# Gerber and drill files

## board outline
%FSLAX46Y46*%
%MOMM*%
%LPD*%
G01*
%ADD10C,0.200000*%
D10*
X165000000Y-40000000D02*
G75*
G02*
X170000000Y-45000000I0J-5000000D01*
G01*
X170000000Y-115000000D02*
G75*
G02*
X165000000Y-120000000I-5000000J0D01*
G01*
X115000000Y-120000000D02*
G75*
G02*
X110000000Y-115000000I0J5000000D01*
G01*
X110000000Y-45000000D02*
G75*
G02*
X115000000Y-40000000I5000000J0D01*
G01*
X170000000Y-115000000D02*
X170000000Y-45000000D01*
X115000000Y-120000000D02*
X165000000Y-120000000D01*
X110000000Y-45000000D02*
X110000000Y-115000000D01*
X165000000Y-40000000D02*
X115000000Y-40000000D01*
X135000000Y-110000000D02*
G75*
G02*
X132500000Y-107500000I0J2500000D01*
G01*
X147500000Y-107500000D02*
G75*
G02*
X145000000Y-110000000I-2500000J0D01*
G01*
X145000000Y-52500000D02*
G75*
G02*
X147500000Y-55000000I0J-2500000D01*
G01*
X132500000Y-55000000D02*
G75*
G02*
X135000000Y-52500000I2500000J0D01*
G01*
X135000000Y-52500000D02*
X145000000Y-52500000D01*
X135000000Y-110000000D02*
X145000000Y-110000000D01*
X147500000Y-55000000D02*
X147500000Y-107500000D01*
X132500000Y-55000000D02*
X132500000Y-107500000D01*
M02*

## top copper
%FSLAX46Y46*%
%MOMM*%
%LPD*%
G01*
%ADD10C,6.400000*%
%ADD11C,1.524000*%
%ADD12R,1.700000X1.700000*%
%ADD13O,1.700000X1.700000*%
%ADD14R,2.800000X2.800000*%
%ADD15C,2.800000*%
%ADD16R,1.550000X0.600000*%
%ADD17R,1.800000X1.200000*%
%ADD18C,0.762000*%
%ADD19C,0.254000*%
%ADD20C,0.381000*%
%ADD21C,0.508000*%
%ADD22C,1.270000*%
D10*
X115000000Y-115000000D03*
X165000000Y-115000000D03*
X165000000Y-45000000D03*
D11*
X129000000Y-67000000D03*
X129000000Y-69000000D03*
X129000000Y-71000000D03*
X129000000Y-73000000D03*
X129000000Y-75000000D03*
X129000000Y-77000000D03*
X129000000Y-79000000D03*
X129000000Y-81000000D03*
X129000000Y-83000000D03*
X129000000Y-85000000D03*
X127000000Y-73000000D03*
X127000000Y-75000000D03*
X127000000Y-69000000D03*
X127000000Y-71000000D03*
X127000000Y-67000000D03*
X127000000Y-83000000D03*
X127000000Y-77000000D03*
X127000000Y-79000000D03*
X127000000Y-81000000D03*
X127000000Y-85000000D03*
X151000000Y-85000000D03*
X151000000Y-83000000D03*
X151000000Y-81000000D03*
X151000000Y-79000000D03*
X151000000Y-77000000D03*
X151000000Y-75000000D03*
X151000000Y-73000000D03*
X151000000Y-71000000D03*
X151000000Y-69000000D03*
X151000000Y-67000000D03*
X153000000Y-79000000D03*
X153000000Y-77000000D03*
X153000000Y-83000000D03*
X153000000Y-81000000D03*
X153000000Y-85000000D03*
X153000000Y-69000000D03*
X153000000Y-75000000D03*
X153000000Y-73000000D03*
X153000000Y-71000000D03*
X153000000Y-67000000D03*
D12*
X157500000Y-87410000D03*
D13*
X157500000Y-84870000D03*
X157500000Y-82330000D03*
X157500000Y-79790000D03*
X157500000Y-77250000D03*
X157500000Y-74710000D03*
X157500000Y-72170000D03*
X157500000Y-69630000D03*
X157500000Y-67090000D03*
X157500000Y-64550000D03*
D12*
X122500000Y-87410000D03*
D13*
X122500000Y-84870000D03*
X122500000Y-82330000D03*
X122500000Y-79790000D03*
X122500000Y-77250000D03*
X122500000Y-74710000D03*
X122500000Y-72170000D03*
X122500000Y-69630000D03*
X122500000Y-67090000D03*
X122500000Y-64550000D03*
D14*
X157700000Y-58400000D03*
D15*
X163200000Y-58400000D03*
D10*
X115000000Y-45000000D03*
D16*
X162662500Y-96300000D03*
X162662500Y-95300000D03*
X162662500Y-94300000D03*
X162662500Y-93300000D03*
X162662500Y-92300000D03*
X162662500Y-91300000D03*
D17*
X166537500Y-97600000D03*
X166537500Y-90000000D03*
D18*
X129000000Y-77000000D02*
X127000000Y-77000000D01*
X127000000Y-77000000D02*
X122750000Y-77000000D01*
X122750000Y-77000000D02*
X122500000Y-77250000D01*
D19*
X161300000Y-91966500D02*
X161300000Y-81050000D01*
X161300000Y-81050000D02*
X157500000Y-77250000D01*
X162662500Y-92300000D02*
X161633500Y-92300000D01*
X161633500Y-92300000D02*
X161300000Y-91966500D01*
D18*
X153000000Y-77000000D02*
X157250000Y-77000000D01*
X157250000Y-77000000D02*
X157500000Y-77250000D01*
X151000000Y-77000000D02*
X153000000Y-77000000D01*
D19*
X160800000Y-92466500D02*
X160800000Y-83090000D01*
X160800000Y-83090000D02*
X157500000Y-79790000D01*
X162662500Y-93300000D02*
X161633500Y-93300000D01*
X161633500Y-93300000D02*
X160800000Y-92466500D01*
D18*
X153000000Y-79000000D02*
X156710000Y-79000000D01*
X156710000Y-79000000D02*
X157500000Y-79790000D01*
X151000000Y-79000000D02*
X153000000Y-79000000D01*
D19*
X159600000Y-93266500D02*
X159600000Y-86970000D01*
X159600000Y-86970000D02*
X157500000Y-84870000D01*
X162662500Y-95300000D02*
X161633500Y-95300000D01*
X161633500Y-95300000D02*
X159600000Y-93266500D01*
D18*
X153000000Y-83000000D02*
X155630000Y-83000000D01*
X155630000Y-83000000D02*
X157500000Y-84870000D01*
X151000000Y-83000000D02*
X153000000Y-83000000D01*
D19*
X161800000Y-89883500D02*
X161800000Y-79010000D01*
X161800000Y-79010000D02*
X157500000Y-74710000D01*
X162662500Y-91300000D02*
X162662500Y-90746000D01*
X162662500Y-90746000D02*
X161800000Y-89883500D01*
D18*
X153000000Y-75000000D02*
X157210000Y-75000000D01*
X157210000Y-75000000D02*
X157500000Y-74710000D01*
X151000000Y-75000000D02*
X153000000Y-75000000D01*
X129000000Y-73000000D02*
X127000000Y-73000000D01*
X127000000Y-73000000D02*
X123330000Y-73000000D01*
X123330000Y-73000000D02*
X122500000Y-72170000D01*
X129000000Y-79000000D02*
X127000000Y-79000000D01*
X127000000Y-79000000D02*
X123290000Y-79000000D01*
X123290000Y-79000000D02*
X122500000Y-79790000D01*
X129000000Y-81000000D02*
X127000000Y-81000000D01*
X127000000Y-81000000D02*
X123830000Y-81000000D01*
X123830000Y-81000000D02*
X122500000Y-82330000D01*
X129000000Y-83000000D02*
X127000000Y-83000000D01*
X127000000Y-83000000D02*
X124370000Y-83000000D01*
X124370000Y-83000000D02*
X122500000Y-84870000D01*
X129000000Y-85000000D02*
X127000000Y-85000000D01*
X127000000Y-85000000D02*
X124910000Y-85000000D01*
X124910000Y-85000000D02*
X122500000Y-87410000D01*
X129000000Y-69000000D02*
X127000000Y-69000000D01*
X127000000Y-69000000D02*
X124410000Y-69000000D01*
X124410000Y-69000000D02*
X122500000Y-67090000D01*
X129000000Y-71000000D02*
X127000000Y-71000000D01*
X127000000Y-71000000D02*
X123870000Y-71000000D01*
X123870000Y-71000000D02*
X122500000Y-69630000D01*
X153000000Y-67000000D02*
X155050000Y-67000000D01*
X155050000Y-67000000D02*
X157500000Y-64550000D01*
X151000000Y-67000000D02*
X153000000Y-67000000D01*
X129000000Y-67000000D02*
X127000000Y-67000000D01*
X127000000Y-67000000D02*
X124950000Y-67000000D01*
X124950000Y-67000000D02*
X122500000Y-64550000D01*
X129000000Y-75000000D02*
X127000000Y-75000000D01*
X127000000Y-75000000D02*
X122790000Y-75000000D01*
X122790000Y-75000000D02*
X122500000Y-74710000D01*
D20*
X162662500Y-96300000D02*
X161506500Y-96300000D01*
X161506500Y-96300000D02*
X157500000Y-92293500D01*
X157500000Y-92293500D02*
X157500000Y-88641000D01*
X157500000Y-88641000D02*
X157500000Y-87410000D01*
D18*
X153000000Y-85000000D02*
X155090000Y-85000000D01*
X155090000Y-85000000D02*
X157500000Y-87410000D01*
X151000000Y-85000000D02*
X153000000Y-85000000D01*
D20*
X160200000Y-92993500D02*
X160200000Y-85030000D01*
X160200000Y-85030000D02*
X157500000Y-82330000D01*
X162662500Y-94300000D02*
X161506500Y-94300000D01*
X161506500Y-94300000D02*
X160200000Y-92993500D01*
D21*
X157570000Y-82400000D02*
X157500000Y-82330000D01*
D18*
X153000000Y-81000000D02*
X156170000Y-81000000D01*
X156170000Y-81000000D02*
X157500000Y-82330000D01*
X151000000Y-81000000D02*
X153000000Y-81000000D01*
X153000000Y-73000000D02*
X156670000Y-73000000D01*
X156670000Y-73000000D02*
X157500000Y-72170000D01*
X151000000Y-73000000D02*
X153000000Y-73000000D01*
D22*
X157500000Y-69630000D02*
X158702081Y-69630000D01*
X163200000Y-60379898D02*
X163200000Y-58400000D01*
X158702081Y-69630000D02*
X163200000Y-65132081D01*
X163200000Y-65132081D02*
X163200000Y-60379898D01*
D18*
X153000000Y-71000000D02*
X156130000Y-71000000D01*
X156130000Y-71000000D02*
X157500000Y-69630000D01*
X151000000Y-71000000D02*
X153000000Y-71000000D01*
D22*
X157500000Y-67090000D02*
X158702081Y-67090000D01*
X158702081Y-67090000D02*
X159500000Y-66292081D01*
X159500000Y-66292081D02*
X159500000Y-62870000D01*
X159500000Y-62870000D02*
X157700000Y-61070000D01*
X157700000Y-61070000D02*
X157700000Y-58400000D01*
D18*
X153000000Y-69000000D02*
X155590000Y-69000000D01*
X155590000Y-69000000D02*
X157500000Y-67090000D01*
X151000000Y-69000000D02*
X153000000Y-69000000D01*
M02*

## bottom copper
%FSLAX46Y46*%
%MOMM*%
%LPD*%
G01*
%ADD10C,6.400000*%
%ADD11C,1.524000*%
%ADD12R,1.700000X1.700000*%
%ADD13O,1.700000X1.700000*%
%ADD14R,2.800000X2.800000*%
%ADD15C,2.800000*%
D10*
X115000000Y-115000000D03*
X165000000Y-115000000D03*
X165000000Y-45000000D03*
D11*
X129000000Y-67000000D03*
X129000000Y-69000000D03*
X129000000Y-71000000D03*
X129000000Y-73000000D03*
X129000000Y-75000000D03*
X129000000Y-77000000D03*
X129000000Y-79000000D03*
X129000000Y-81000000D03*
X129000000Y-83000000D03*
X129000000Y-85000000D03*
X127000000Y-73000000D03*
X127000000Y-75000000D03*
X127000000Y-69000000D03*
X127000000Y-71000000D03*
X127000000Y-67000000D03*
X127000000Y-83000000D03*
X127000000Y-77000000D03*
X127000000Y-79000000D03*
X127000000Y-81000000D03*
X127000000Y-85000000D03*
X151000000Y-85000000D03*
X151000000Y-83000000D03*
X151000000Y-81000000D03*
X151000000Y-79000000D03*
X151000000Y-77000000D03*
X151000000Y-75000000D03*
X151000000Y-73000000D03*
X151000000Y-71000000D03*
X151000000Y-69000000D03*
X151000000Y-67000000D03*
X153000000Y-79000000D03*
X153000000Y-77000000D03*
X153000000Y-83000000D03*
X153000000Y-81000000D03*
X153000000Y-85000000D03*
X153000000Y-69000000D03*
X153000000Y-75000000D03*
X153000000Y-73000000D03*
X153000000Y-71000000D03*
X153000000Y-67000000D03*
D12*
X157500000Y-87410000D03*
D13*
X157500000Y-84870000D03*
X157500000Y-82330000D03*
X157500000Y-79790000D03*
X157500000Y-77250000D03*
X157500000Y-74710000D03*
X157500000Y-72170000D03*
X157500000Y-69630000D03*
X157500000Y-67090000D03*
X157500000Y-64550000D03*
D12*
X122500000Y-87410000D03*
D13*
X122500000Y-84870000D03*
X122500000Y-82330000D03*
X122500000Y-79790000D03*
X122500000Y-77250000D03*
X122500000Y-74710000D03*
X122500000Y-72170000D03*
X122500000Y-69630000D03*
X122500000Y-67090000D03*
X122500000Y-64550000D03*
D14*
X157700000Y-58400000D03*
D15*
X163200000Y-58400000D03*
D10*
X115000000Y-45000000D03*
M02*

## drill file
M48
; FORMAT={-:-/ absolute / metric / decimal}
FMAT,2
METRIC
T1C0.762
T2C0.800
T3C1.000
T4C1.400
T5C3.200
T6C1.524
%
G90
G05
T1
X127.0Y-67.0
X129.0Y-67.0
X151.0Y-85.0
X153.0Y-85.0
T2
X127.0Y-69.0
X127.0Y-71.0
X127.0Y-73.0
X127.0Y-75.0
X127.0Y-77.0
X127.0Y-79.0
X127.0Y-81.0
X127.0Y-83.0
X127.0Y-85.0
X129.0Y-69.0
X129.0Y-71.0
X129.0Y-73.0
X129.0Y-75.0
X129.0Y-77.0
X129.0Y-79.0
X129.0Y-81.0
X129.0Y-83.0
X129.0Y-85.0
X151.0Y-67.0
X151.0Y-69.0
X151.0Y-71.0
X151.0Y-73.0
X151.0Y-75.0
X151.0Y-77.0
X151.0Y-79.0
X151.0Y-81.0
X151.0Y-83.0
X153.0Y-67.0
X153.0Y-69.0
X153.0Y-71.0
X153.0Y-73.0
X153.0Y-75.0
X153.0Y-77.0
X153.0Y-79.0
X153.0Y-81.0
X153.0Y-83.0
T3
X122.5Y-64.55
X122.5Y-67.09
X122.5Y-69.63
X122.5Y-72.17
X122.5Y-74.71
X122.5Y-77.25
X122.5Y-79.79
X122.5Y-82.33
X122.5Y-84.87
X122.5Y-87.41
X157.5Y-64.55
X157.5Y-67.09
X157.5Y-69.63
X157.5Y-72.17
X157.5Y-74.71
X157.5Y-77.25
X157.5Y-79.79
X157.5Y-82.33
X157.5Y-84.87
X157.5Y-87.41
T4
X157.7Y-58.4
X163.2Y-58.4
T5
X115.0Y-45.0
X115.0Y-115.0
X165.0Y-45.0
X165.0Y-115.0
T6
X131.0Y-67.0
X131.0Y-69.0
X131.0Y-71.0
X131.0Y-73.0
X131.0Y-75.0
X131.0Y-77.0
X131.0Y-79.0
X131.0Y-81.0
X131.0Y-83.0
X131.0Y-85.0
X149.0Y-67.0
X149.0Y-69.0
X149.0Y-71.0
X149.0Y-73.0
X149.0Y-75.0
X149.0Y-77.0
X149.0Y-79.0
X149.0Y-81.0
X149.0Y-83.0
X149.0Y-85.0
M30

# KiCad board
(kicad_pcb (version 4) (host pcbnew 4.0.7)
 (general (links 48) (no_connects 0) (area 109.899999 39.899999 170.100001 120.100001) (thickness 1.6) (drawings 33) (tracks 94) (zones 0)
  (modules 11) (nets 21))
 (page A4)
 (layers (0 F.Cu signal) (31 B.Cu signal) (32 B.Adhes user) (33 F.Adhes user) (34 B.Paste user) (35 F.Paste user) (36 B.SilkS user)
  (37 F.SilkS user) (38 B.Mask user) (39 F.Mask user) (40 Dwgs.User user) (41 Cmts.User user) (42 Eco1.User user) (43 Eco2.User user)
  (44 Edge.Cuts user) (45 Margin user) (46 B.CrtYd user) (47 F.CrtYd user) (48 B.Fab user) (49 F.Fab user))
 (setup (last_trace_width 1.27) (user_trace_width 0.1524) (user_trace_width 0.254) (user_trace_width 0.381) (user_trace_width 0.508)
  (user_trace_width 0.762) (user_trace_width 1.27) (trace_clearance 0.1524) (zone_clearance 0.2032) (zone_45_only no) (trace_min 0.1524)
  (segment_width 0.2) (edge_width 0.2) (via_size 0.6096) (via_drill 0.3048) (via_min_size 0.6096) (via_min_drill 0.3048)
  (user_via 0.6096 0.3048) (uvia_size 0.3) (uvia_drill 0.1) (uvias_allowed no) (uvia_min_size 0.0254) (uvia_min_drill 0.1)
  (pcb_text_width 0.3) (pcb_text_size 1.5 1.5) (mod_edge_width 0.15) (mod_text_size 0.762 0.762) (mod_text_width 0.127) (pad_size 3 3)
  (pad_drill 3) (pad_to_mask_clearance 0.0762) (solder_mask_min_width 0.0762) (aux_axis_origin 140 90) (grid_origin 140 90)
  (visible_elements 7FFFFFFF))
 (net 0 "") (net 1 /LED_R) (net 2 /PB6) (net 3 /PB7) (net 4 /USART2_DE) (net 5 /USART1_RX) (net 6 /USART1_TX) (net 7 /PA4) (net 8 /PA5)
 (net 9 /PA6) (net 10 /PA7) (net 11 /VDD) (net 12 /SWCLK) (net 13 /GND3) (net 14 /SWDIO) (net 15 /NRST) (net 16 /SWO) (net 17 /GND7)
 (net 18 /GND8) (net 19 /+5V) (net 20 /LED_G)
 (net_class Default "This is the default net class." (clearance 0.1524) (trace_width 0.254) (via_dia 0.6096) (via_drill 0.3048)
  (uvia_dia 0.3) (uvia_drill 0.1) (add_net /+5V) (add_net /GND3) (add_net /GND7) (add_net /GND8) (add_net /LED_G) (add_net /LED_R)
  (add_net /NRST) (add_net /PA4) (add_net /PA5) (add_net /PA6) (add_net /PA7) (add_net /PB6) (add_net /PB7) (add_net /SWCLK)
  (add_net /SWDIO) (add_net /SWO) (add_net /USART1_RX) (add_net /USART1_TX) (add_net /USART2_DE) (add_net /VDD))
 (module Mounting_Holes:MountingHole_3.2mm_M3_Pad (layer F.Cu) (at 115 115)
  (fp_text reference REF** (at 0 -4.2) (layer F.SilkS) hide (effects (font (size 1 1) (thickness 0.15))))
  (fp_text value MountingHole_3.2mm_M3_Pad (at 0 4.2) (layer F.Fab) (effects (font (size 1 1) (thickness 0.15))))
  (pad 1 thru_hole circle (at 0 0) (size 6.4 6.4) (drill 3.2) (layers *.Cu *.Mask)))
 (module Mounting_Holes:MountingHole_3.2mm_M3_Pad (layer F.Cu) (at 165 115)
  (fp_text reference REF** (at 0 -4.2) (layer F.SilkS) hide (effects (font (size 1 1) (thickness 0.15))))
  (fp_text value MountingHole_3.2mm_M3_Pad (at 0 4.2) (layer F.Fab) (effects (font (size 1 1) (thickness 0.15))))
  (pad 1 thru_hole circle (at 0 0) (size 6.4 6.4) (drill 3.2) (layers *.Cu *.Mask)))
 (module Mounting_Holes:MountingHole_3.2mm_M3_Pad (layer F.Cu) (at 165 45)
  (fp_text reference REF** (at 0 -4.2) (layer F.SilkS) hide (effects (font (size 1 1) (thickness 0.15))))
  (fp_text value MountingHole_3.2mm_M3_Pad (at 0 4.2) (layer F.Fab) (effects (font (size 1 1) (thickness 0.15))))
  (pad 1 thru_hole circle (at 0 0) (size 6.4 6.4) (drill 3.2) (layers *.Cu *.Mask)))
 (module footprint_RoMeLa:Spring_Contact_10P (layer F.Cu) (at 129 67 180)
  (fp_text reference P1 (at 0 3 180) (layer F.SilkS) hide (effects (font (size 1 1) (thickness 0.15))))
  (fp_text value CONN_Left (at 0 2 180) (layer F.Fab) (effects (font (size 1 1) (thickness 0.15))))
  (pad 1 thru_hole circle (at 0 0 180) (size 1.524 1.524) (drill 0.762) (layers *.Cu *.Mask) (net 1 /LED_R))
  (pad 2 thru_hole circle (at 0 -2 180) (size 1.524 1.524) (drill 0.8) (layers *.Cu *.Mask) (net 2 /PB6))
  (pad 3 thru_hole circle (at 0 -4 180) (size 1.524 1.524) (drill 0.8) (layers *.Cu *.Mask) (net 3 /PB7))
  (pad 4 thru_hole circle (at 0 -6 180) (size 1.524 1.524) (drill 0.8) (layers *.Cu *.Mask) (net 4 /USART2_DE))
  (pad 5 thru_hole circle (at 0 -8 180) (size 1.524 1.524) (drill 0.8) (layers *.Cu *.Mask) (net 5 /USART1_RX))
  (pad 6 thru_hole circle (at 0 -10 180) (size 1.524 1.524) (drill 0.8) (layers *.Cu *.Mask) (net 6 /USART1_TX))
  (pad 7 thru_hole circle (at 0 -12 180) (size 1.524 1.524) (drill 0.8) (layers *.Cu *.Mask) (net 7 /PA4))
  (pad 8 thru_hole circle (at 0 -14 180) (size 1.524 1.524) (drill 0.8) (layers *.Cu *.Mask) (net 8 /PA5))
  (pad 9 thru_hole circle (at 0 -16 180) (size 1.524 1.524) (drill 0.8) (layers *.Cu *.Mask) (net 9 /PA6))
  (pad 10 thru_hole circle (at 0 -18 180) (size 1.524 1.524) (drill 0.8) (layers *.Cu *.Mask) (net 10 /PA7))
  (pad 4 thru_hole circle (at 2 -6 180) (size 1.524 1.524) (drill 0.8) (layers *.Cu *.Mask) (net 4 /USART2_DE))
  (pad 5 thru_hole circle (at 2 -8 180) (size 1.524 1.524) (drill 0.8) (layers *.Cu *.Mask) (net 5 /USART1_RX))
  (pad 2 thru_hole circle (at 2 -2 180) (size 1.524 1.524) (drill 0.8) (layers *.Cu *.Mask) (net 2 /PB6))
  (pad 3 thru_hole circle (at 2 -4 180) (size 1.524 1.524) (drill 0.8) (layers *.Cu *.Mask) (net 3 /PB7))
  (pad 1 thru_hole circle (at 2 0 180) (size 1.524 1.524) (drill 0.762) (layers *.Cu *.Mask) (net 1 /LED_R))
  (pad 9 thru_hole circle (at 2 -16 180) (size 1.524 1.524) (drill 0.8) (layers *.Cu *.Mask) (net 9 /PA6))
  (pad 6 thru_hole circle (at 2 -10 180) (size 1.524 1.524) (drill 0.8) (layers *.Cu *.Mask) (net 6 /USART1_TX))
  (pad 7 thru_hole circle (at 2 -12 180) (size 1.524 1.524) (drill 0.8) (layers *.Cu *.Mask) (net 7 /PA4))
  (pad 8 thru_hole circle (at 2 -14 180) (size 1.524 1.524) (drill 0.8) (layers *.Cu *.Mask) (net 8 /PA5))
  (pad 10 thru_hole circle (at 2 -18 180) (size 1.524 1.524) (drill 0.8) (layers *.Cu *.Mask) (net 10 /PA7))
  (pad "" np_thru_hole circle (at -2 0 180) (size 1.524 1.524) (drill 1.524) (layers *.Cu *.Mask))
  (pad "" np_thru_hole circle (at -2 -2 180) (size 1.524 1.524) (drill 1.524) (layers *.Cu *.Mask))
  (pad "" np_thru_hole circle (at -2 -4 180) (size 1.524 1.524) (drill 1.524) (layers *.Cu *.Mask))
  (pad "" np_thru_hole circle (at -2 -6 180) (size 1.524 1.524) (drill 1.524) (layers *.Cu *.Mask))
  (pad "" np_thru_hole circle (at -2 -8 180) (size 1.524 1.524) (drill 1.524) (layers *.Cu *.Mask))
  (pad "" np_thru_hole circle (at -2 -10 180) (size 1.524 1.524) (drill 1.524) (layers *.Cu *.Mask))
  (pad "" np_thru_hole circle (at -2 -12 180) (size 1.524 1.524) (drill 1.524) (layers *.Cu *.Mask))
  (pad "" np_thru_hole circle (at -2 -14 180) (size 1.524 1.524) (drill 1.524) (layers *.Cu *.Mask))
  (pad "" np_thru_hole circle (at -2 -16 180) (size 1.524 1.524) (drill 1.524) (layers *.Cu *.Mask))
  (pad "" np_thru_hole circle (at -2 -18 180) (size 1.524 1.524) (drill 1.524) (layers *.Cu *.Mask)))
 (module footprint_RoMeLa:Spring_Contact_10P (layer F.Cu) (at 151 85)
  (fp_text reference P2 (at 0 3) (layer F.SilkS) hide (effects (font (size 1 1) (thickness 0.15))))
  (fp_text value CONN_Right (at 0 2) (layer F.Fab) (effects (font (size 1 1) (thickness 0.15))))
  (pad 1 thru_hole circle (at 0 0) (size 1.524 1.524) (drill 0.762) (layers *.Cu *.Mask) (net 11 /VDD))
  (pad 2 thru_hole circle (at 0 -2) (size 1.524 1.524) (drill 0.8) (layers *.Cu *.Mask) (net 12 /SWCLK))
  (pad 3 thru_hole circle (at 0 -4) (size 1.524 1.524) (drill 0.8) (layers *.Cu *.Mask) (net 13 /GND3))
  (pad 4 thru_hole circle (at 0 -6) (size 1.524 1.524) (drill 0.8) (layers *.Cu *.Mask) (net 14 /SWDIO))
  (pad 5 thru_hole circle (at 0 -8) (size 1.524 1.524) (drill 0.8) (layers *.Cu *.Mask) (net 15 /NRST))
  (pad 6 thru_hole circle (at 0 -10) (size 1.524 1.524) (drill 0.8) (layers *.Cu *.Mask) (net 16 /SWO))
  (pad 7 thru_hole circle (at 0 -12) (size 1.524 1.524) (drill 0.8) (layers *.Cu *.Mask) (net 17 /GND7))
  (pad 8 thru_hole circle (at 0 -14) (size 1.524 1.524) (drill 0.8) (layers *.Cu *.Mask) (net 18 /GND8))
  (pad 9 thru_hole circle (at 0 -16) (size 1.524 1.524) (drill 0.8) (layers *.Cu *.Mask) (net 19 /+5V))
  (pad 10 thru_hole circle (at 0 -18) (size 1.524 1.524) (drill 0.8) (layers *.Cu *.Mask) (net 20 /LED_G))
  (pad 4 thru_hole circle (at 2 -6) (size 1.524 1.524) (drill 0.8) (layers *.Cu *.Mask) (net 14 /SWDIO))
  (pad 5 thru_hole circle (at 2 -8) (size 1.524 1.524) (drill 0.8) (layers *.Cu *.Mask) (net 15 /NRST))
  (pad 2 thru_hole circle (at 2 -2) (size 1.524 1.524) (drill 0.8) (layers *.Cu *.Mask) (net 12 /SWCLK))
  (pad 3 thru_hole circle (at 2 -4) (size 1.524 1.524) (drill 0.8) (layers *.Cu *.Mask) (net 13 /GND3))
  (pad 1 thru_hole circle (at 2 0) (size 1.524 1.524) (drill 0.762) (layers *.Cu *.Mask) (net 11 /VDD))
  (pad 9 thru_hole circle (at 2 -16) (size 1.524 1.524) (drill 0.8) (layers *.Cu *.Mask) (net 19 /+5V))
  (pad 6 thru_hole circle (at 2 -10) (size 1.524 1.524) (drill 0.8) (layers *.Cu *.Mask) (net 16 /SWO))
  (pad 7 thru_hole circle (at 2 -12) (size 1.524 1.524) (drill 0.8) (layers *.Cu *.Mask) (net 17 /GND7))
  (pad 8 thru_hole circle (at 2 -14) (size 1.524 1.524) (drill 0.8) (layers *.Cu *.Mask) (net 18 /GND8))
  (pad 10 thru_hole circle (at 2 -18) (size 1.524 1.524) (drill 0.8) (layers *.Cu *.Mask) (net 20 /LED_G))
  (pad "" np_thru_hole circle (at -2 0) (size 1.524 1.524) (drill 1.524) (layers *.Cu *.Mask))
  (pad "" np_thru_hole circle (at -2 -2) (size 1.524 1.524) (drill 1.524) (layers *.Cu *.Mask))
  (pad "" np_thru_hole circle (at -2 -4) (size 1.524 1.524) (drill 1.524) (layers *.Cu *.Mask))
  (pad "" np_thru_hole circle (at -2 -6) (size 1.524 1.524) (drill 1.524) (layers *.Cu *.Mask))
  (pad "" np_thru_hole circle (at -2 -8) (size 1.524 1.524) (drill 1.524) (layers *.Cu *.Mask))
  (pad "" np_thru_hole circle (at -2 -10) (size 1.524 1.524) (drill 1.524) (layers *.Cu *.Mask))
  (pad "" np_thru_hole circle (at -2 -12) (size 1.524 1.524) (drill 1.524) (layers *.Cu *.Mask))
  (pad "" np_thru_hole circle (at -2 -14) (size 1.524 1.524) (drill 1.524) (layers *.Cu *.Mask))
  (pad "" np_thru_hole circle (at -2 -16) (size 1.524 1.524) (drill 1.524) (layers *.Cu *.Mask))
  (pad "" np_thru_hole circle (at -2 -18) (size 1.524 1.524) (drill 1.524) (layers *.Cu *.Mask)))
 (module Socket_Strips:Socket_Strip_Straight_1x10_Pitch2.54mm (layer F.Cu) (at 157.5 87.41 180)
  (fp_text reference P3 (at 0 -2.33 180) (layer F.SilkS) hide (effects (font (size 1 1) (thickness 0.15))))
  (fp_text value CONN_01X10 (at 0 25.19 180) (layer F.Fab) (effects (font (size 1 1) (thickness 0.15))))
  (pad 1 thru_hole rect (at 0 0 180) (size 1.7 1.7) (drill 1) (layers *.Cu *.Mask) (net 11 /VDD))
  (pad 2 thru_hole oval (at 0 2.54 180) (size 1.7 1.7) (drill 1) (layers *.Cu *.Mask) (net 12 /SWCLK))
  (pad 3 thru_hole oval (at 0 5.08 180) (size 1.7 1.7) (drill 1) (layers *.Cu *.Mask) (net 13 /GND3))
  (pad 4 thru_hole oval (at 0 7.62 180) (size 1.7 1.7) (drill 1) (layers *.Cu *.Mask) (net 14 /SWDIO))
  (pad 5 thru_hole oval (at 0 10.16 180) (size 1.7 1.7) (drill 1) (layers *.Cu *.Mask) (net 15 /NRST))
  (pad 6 thru_hole oval (at 0 12.7 180) (size 1.7 1.7) (drill 1) (layers *.Cu *.Mask) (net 16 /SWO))
  (pad 7 thru_hole oval (at 0 15.24 180) (size 1.7 1.7) (drill 1) (layers *.Cu *.Mask) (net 17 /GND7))
  (pad 8 thru_hole oval (at 0 17.78 180) (size 1.7 1.7) (drill 1) (layers *.Cu *.Mask) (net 18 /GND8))
  (pad 9 thru_hole oval (at 0 20.32 180) (size 1.7 1.7) (drill 1) (layers *.Cu *.Mask) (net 19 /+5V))
  (pad 10 thru_hole oval (at 0 22.86 180) (size 1.7 1.7) (drill 1) (layers *.Cu *.Mask) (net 20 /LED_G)))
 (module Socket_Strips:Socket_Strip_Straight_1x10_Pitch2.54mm (layer F.Cu) (at 122.5 87.41 180)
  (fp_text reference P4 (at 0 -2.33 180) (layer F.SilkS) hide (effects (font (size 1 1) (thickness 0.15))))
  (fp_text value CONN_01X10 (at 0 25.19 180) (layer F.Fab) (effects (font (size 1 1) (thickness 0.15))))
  (pad 1 thru_hole rect (at 0 0 180) (size 1.7 1.7) (drill 1) (layers *.Cu *.Mask) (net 10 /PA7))
  (pad 2 thru_hole oval (at 0 2.54 180) (size 1.7 1.7) (drill 1) (layers *.Cu *.Mask) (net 9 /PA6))
  (pad 3 thru_hole oval (at 0 5.08 180) (size 1.7 1.7) (drill 1) (layers *.Cu *.Mask) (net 8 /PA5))
  (pad 4 thru_hole oval (at 0 7.62 180) (size 1.7 1.7) (drill 1) (layers *.Cu *.Mask) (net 7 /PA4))
  (pad 5 thru_hole oval (at 0 10.16 180) (size 1.7 1.7) (drill 1) (layers *.Cu *.Mask) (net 6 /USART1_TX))
  (pad 6 thru_hole oval (at 0 12.7 180) (size 1.7 1.7) (drill 1) (layers *.Cu *.Mask) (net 5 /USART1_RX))
  (pad 7 thru_hole oval (at 0 15.24 180) (size 1.7 1.7) (drill 1) (layers *.Cu *.Mask) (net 4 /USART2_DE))
  (pad 8 thru_hole oval (at 0 17.78 180) (size 1.7 1.7) (drill 1) (layers *.Cu *.Mask) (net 3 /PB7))
  (pad 9 thru_hole oval (at 0 20.32 180) (size 1.7 1.7) (drill 1) (layers *.Cu *.Mask) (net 2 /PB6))
  (pad 10 thru_hole oval (at 0 22.86 180) (size 1.7 1.7) (drill 1) (layers *.Cu *.Mask) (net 1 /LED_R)))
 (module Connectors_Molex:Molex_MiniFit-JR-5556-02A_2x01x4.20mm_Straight (layer F.Cu) (at 157.7 58.4 90)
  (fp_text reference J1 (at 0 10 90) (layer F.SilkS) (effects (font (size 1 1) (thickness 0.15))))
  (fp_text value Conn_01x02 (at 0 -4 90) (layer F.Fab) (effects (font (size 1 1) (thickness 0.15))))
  (pad 1 thru_hole rect (at 0 0 90) (size 2.8 2.8) (drill 1.4) (layers *.Cu *.Mask) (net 19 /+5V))
  (pad 2 thru_hole circle (at 0 5.5 90) (size 2.8 2.8) (drill 1.4) (layers *.Cu *.Mask) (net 18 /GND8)))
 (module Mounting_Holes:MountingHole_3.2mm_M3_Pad (layer F.Cu) (at 115 45)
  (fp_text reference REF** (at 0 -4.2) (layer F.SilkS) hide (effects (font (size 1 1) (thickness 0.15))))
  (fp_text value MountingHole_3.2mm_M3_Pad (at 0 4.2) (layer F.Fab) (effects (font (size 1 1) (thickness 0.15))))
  (pad 1 thru_hole circle (at 0 0) (size 6.4 6.4) (drill 3.2) (layers *.Cu *.Mask)))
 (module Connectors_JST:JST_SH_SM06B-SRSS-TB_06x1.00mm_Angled (layer F.Cu) (at 164.6 93.8 90)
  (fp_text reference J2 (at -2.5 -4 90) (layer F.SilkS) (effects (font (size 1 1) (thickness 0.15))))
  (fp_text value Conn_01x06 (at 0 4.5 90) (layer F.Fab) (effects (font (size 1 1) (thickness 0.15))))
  (pad 1 smd rect (at -2.5 -1.9375 90) (size 0.6 1.55) (layers F.Cu F.Paste F.Mask) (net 11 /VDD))
  (pad 2 smd rect (at -1.5 -1.9375 90) (size 0.6 1.55) (layers F.Cu F.Paste F.Mask) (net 12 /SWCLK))
  (pad 3 smd rect (at -0.5 -1.9375 90) (size 0.6 1.55) (layers F.Cu F.Paste F.Mask) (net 13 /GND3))
  (pad 4 smd rect (at 0.5 -1.9375 90) (size 0.6 1.55) (layers F.Cu F.Paste F.Mask) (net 14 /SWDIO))
  (pad 5 smd rect (at 1.5 -1.9375 90) (size 0.6 1.55) (layers F.Cu F.Paste F.Mask) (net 15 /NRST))
  (pad 6 smd rect (at 2.5 -1.9375 90) (size 0.6 1.55) (layers F.Cu F.Paste F.Mask) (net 16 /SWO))
  (pad "" smd rect (at -3.8 1.9375 90) (size 1.2 1.8) (layers F.Cu F.Paste F.Mask))
  (pad "" smd rect (at 3.8 1.9375 90) (size 1.2 1.8) (layers F.Cu F.Paste F.Mask)))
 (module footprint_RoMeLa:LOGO (layer F.Cu) (at 153.9 106.7)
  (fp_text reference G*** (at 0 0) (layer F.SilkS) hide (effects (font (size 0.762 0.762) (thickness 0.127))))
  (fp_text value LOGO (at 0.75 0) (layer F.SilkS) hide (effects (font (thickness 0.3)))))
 (gr_arc (start 165 45) (end 165 40) (angle 90) (layer Edge.Cuts) (width 0.2))
 (gr_arc (start 165 115) (end 170 115) (angle 90) (layer Edge.Cuts) (width 0.2))
 (gr_arc (start 115 115) (end 115 120) (angle 90) (layer Edge.Cuts) (width 0.2))
 (gr_arc (start 115 45) (end 110 45) (angle 90) (layer Edge.Cuts) (width 0.2))
 (gr_line (start 170 115) (end 170 45) (layer Edge.Cuts) (width 0.2))
 (gr_line (start 115 120) (end 165 120) (layer Edge.Cuts) (width 0.2))
 (gr_line (start 110 45) (end 110 115) (layer Edge.Cuts) (width 0.2))
 (gr_line (start 165 40) (end 115 40) (layer Edge.Cuts) (width 0.2))
 (gr_arc (start 135 107.5) (end 135 110) (angle 90) (layer Edge.Cuts) (width 0.2))
 (gr_arc (start 145 107.5) (end 147.5 107.5) (angle 90) (layer Edge.Cuts) (width 0.2))
 (gr_arc (start 145 55) (end 145 52.5) (angle 90) (layer Edge.Cuts) (width 0.2))
 (gr_arc (start 135 55) (end 132.5 55) (angle 90) (layer Edge.Cuts) (width 0.2))
 (gr_line (start 135 52.5) (end 145 52.5) (layer Edge.Cuts) (width 0.2))
 (gr_line (start 135 110) (end 145 110) (layer Edge.Cuts) (width 0.2))
 (gr_line (start 147.5 55) (end 147.5 107.5) (layer Edge.Cuts) (width 0.2))
 (gr_line (start 132.5 55) (end 132.5 107.5) (layer Edge.Cuts) (width 0.2))
 (segment (start 129 77) (end 127 77) (width 0.762) (layer F.Cu) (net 6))
 (segment (start 127 77) (end 122.75 77) (width 0.762) (layer F.Cu) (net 6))
 (segment (start 122.75 77) (end 122.5 77.25) (width 0.762) (layer F.Cu) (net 6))
 (segment (start 161.3 91.9665) (end 161.3 81.05) (width 0.254) (layer F.Cu) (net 15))
 (segment (start 161.3 81.05) (end 157.5 77.25) (width 0.254) (layer F.Cu) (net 15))
 (segment (start 162.6625 92.3) (end 161.6335 92.3) (width 0.254) (layer F.Cu) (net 15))
 (segment (start 161.6335 92.3) (end 161.3 91.9665) (width 0.254) (layer F.Cu) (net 15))
 (segment (start 153 77) (end 157.25 77) (width 0.762) (layer F.Cu) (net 15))
 (segment (start 157.25 77) (end 157.5 77.25) (width 0.762) (layer F.Cu) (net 15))
 (segment (start 151 77) (end 153 77) (width 0.762) (layer F.Cu) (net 15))
 (segment (start 160.8 92.4665) (end 160.8 83.09) (width 0.254) (layer F.Cu) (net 14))
 (segment (start 160.8 83.09) (end 157.5 79.79) (width 0.254) (layer F.Cu) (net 14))
 (segment (start 162.6625 93.3) (end 161.6335 93.3) (width 0.254) (layer F.Cu) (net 14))
 (segment (start 161.6335 93.3) (end 160.8 92.4665) (width 0.254) (layer F.Cu) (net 14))
 (segment (start 153 79) (end 156.71 79) (width 0.762) (layer F.Cu) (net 14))
 (segment (start 156.71 79) (end 157.5 79.79) (width 0.762) (layer F.Cu) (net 14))
 (segment (start 151 79) (end 153 79) (width 0.762) (layer F.Cu) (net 14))
 (segment (start 159.6 93.2665) (end 159.6 86.97) (width 0.254) (layer F.Cu) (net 12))
 (segment (start 159.6 86.97) (end 157.5 84.87) (width 0.254) (layer F.Cu) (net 12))
 (segment (start 162.6625 95.3) (end 161.6335 95.3) (width 0.254) (layer F.Cu) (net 12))
 (segment (start 161.6335 95.3) (end 159.6 93.2665) (width 0.254) (layer F.Cu) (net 12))
 (segment (start 153 83) (end 155.63 83) (width 0.762) (layer F.Cu) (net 12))
 (segment (start 155.63 83) (end 157.5 84.87) (width 0.762) (layer F.Cu) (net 12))
 (segment (start 151 83) (end 153 83) (width 0.762) (layer F.Cu) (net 12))
 (segment (start 161.8 89.8835) (end 161.8 79.01) (width 0.254) (layer F.Cu) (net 16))
 (segment (start 161.8 79.01) (end 157.5 74.71) (width 0.254) (layer F.Cu) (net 16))
 (segment (start 162.6625 91.3) (end 162.6625 90.746) (width 0.254) (layer F.Cu) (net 16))
 (segment (start 162.6625 90.746) (end 161.8 89.8835) (width 0.254) (layer F.Cu) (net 16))
 (segment (start 153 75) (end 157.21 75) (width 0.762) (layer F.Cu) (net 16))
 (segment (start 157.21 75) (end 157.5 74.71) (width 0.762) (layer F.Cu) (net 16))
 (segment (start 151 75) (end 153 75) (width 0.762) (layer F.Cu) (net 16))
 (segment (start 129 73) (end 127 73) (width 0.762) (layer F.Cu) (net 4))
 (segment (start 127 73) (end 123.33 73) (width 0.762) (layer F.Cu) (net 4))
 (segment (start 123.33 73) (end 122.5 72.17) (width 0.762) (layer F.Cu) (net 4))
 (segment (start 129 79) (end 127 79) (width 0.762) (layer F.Cu) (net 7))
 (segment (start 127 79) (end 123.29 79) (width 0.762) (layer F.Cu) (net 7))
 (segment (start 123.29 79) (end 122.5 79.79) (width 0.762) (layer F.Cu) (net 7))
 (segment (start 129 81) (end 127 81) (width 0.762) (layer F.Cu) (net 8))
 (segment (start 127 81) (end 123.83 81) (width 0.762) (layer F.Cu) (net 8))
 (segment (start 123.83 81) (end 122.5 82.33) (width 0.762) (layer F.Cu) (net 8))
 (segment (start 129 83) (end 127 83) (width 0.762) (layer F.Cu) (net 9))
 (segment (start 127 83) (end 124.37 83) (width 0.762) (layer F.Cu) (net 9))
 (segment (start 124.37 83) (end 122.5 84.87) (width 0.762) (layer F.Cu) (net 9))
 (segment (start 129 85) (end 127 85) (width 0.762) (layer F.Cu) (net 10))
 (segment (start 127 85) (end 124.91 85) (width 0.762) (layer F.Cu) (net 10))
 (segment (start 124.91 85) (end 122.5 87.41) (width 0.762) (layer F.Cu) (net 10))
 (segment (start 129 69) (end 127 69) (width 0.762) (layer F.Cu) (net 2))
 (segment (start 127 69) (end 124.41 69) (width 0.762) (layer F.Cu) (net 2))
 (segment (start 124.41 69) (end 122.5 67.09) (width 0.762) (layer F.Cu) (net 2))
 (segment (start 129 71) (end 127 71) (width 0.762) (layer F.Cu) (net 3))
 (segment (start 127 71) (end 123.87 71) (width 0.762) (layer F.Cu) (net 3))
 (segment (start 123.87 71) (end 122.5 69.63) (width 0.762) (layer F.Cu) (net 3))
 (segment (start 153 67) (end 155.05 67) (width 0.762) (layer F.Cu) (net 20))
 (segment (start 155.05 67) (end 157.5 64.55) (width 0.762) (layer F.Cu) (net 20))
 (segment (start 151 67) (end 153 67) (width 0.762) (layer F.Cu) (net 20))
 (segment (start 129 67) (end 127 67) (width 0.762) (layer F.Cu) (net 1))
 (segment (start 127 67) (end 124.95 67) (width 0.762) (layer F.Cu) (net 1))
 (segment (start 124.95 67) (end 122.5 64.55) (width 0.762) (layer F.Cu) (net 1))
 (segment (start 129 75) (end 127 75) (width 0.762) (layer F.Cu) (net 5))
 (segment (start 127 75) (end 122.79 75) (width 0.762) (layer F.Cu) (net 5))
 (segment (start 122.79 75) (end 122.5 74.71) (width 0.762) (layer F.Cu) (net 5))
 (segment (start 162.6625 96.3) (end 161.5065 96.3) (width 0.381) (layer F.Cu) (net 11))
 (segment (start 161.5065 96.3) (end 157.5 92.2935) (width 0.381) (layer F.Cu) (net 11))
 (segment (start 157.5 92.2935) (end 157.5 88.641) (width 0.381) (layer F.Cu) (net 11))
 (segment (start 157.5 88.641) (end 157.5 87.41) (width 0.381) (layer F.Cu) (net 11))
 (segment (start 153 85) (end 155.09 85) (width 0.762) (layer F.Cu) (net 11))
 (segment (start 155.09 85) (end 157.5 87.41) (width 0.762) (layer F.Cu) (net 11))
 (segment (start 151 85) (end 153 85) (width 0.762) (layer F.Cu) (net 11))
 (segment (start 160.2 92.9935) (end 160.2 85.03) (width 0.381) (layer F.Cu) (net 13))
 (segment (start 160.2 85.03) (end 157.5 82.33) (width 0.381) (layer F.Cu) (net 13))
 (segment (start 162.6625 94.3) (end 161.5065 94.3) (width 0.381) (layer F.Cu) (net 13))
 (segment (start 161.5065 94.3) (end 160.2 92.9935) (width 0.381) (layer F.Cu) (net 13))
 (segment (start 157.57 82.4) (end 157.5 82.33) (width 0.508) (layer F.Cu) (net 13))
 (segment (start 153 81) (end 156.17 81) (width 0.762) (layer F.Cu) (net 13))
 (segment (start 156.17 81) (end 157.5 82.33) (width 0.762) (layer F.Cu) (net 13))
 (segment (start 151 81) (end 153 81) (width 0.762) (layer F.Cu) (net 13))
 (segment (start 153 73) (end 156.67 73) (width 0.762) (layer F.Cu) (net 17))
 (segment (start 156.67 73) (end 157.5 72.17) (width 0.762) (layer F.Cu) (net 17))
 (segment (start 151 73) (end 153 73) (width 0.762) (layer F.Cu) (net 17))
 (segment (start 157.5 69.63) (end 158.702081 69.63) (width 1.27) (layer F.Cu) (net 18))
 (segment (start 163.2 60.379898) (end 163.2 58.4) (width 1.27) (layer F.Cu) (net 18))
 (segment (start 158.702081 69.63) (end 163.2 65.132081) (width 1.27) (layer F.Cu) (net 18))
 (segment (start 163.2 65.132081) (end 163.2 60.379898) (width 1.27) (layer F.Cu) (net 18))
 (segment (start 153 71) (end 156.13 71) (width 0.762) (layer F.Cu) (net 18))
 (segment (start 156.13 71) (end 157.5 69.63) (width 0.762) (layer F.Cu) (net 18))
 (segment (start 151 71) (end 153 71) (width 0.762) (layer F.Cu) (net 18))
 (segment (start 157.5 67.09) (end 158.702081 67.09) (width 1.27) (layer F.Cu) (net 19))
 (segment (start 158.702081 67.09) (end 159.5 66.292081) (width 1.27) (layer F.Cu) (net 19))
 (segment (start 159.5 66.292081) (end 159.5 62.87) (width 1.27) (layer F.Cu) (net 19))
 (segment (start 159.5 62.87) (end 157.7 61.07) (width 1.27) (layer F.Cu) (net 19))
 (segment (start 157.7 61.07) (end 157.7 58.4) (width 1.27) (layer F.Cu) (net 19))
 (segment (start 153 69) (end 155.59 69) (width 0.762) (layer F.Cu) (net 19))
 (segment (start 155.59 69) (end 157.5 67.09) (width 0.762) (layer F.Cu) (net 19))
 (segment (start 151 69) (end 153 69) (width 0.762) (layer F.Cu) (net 19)))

